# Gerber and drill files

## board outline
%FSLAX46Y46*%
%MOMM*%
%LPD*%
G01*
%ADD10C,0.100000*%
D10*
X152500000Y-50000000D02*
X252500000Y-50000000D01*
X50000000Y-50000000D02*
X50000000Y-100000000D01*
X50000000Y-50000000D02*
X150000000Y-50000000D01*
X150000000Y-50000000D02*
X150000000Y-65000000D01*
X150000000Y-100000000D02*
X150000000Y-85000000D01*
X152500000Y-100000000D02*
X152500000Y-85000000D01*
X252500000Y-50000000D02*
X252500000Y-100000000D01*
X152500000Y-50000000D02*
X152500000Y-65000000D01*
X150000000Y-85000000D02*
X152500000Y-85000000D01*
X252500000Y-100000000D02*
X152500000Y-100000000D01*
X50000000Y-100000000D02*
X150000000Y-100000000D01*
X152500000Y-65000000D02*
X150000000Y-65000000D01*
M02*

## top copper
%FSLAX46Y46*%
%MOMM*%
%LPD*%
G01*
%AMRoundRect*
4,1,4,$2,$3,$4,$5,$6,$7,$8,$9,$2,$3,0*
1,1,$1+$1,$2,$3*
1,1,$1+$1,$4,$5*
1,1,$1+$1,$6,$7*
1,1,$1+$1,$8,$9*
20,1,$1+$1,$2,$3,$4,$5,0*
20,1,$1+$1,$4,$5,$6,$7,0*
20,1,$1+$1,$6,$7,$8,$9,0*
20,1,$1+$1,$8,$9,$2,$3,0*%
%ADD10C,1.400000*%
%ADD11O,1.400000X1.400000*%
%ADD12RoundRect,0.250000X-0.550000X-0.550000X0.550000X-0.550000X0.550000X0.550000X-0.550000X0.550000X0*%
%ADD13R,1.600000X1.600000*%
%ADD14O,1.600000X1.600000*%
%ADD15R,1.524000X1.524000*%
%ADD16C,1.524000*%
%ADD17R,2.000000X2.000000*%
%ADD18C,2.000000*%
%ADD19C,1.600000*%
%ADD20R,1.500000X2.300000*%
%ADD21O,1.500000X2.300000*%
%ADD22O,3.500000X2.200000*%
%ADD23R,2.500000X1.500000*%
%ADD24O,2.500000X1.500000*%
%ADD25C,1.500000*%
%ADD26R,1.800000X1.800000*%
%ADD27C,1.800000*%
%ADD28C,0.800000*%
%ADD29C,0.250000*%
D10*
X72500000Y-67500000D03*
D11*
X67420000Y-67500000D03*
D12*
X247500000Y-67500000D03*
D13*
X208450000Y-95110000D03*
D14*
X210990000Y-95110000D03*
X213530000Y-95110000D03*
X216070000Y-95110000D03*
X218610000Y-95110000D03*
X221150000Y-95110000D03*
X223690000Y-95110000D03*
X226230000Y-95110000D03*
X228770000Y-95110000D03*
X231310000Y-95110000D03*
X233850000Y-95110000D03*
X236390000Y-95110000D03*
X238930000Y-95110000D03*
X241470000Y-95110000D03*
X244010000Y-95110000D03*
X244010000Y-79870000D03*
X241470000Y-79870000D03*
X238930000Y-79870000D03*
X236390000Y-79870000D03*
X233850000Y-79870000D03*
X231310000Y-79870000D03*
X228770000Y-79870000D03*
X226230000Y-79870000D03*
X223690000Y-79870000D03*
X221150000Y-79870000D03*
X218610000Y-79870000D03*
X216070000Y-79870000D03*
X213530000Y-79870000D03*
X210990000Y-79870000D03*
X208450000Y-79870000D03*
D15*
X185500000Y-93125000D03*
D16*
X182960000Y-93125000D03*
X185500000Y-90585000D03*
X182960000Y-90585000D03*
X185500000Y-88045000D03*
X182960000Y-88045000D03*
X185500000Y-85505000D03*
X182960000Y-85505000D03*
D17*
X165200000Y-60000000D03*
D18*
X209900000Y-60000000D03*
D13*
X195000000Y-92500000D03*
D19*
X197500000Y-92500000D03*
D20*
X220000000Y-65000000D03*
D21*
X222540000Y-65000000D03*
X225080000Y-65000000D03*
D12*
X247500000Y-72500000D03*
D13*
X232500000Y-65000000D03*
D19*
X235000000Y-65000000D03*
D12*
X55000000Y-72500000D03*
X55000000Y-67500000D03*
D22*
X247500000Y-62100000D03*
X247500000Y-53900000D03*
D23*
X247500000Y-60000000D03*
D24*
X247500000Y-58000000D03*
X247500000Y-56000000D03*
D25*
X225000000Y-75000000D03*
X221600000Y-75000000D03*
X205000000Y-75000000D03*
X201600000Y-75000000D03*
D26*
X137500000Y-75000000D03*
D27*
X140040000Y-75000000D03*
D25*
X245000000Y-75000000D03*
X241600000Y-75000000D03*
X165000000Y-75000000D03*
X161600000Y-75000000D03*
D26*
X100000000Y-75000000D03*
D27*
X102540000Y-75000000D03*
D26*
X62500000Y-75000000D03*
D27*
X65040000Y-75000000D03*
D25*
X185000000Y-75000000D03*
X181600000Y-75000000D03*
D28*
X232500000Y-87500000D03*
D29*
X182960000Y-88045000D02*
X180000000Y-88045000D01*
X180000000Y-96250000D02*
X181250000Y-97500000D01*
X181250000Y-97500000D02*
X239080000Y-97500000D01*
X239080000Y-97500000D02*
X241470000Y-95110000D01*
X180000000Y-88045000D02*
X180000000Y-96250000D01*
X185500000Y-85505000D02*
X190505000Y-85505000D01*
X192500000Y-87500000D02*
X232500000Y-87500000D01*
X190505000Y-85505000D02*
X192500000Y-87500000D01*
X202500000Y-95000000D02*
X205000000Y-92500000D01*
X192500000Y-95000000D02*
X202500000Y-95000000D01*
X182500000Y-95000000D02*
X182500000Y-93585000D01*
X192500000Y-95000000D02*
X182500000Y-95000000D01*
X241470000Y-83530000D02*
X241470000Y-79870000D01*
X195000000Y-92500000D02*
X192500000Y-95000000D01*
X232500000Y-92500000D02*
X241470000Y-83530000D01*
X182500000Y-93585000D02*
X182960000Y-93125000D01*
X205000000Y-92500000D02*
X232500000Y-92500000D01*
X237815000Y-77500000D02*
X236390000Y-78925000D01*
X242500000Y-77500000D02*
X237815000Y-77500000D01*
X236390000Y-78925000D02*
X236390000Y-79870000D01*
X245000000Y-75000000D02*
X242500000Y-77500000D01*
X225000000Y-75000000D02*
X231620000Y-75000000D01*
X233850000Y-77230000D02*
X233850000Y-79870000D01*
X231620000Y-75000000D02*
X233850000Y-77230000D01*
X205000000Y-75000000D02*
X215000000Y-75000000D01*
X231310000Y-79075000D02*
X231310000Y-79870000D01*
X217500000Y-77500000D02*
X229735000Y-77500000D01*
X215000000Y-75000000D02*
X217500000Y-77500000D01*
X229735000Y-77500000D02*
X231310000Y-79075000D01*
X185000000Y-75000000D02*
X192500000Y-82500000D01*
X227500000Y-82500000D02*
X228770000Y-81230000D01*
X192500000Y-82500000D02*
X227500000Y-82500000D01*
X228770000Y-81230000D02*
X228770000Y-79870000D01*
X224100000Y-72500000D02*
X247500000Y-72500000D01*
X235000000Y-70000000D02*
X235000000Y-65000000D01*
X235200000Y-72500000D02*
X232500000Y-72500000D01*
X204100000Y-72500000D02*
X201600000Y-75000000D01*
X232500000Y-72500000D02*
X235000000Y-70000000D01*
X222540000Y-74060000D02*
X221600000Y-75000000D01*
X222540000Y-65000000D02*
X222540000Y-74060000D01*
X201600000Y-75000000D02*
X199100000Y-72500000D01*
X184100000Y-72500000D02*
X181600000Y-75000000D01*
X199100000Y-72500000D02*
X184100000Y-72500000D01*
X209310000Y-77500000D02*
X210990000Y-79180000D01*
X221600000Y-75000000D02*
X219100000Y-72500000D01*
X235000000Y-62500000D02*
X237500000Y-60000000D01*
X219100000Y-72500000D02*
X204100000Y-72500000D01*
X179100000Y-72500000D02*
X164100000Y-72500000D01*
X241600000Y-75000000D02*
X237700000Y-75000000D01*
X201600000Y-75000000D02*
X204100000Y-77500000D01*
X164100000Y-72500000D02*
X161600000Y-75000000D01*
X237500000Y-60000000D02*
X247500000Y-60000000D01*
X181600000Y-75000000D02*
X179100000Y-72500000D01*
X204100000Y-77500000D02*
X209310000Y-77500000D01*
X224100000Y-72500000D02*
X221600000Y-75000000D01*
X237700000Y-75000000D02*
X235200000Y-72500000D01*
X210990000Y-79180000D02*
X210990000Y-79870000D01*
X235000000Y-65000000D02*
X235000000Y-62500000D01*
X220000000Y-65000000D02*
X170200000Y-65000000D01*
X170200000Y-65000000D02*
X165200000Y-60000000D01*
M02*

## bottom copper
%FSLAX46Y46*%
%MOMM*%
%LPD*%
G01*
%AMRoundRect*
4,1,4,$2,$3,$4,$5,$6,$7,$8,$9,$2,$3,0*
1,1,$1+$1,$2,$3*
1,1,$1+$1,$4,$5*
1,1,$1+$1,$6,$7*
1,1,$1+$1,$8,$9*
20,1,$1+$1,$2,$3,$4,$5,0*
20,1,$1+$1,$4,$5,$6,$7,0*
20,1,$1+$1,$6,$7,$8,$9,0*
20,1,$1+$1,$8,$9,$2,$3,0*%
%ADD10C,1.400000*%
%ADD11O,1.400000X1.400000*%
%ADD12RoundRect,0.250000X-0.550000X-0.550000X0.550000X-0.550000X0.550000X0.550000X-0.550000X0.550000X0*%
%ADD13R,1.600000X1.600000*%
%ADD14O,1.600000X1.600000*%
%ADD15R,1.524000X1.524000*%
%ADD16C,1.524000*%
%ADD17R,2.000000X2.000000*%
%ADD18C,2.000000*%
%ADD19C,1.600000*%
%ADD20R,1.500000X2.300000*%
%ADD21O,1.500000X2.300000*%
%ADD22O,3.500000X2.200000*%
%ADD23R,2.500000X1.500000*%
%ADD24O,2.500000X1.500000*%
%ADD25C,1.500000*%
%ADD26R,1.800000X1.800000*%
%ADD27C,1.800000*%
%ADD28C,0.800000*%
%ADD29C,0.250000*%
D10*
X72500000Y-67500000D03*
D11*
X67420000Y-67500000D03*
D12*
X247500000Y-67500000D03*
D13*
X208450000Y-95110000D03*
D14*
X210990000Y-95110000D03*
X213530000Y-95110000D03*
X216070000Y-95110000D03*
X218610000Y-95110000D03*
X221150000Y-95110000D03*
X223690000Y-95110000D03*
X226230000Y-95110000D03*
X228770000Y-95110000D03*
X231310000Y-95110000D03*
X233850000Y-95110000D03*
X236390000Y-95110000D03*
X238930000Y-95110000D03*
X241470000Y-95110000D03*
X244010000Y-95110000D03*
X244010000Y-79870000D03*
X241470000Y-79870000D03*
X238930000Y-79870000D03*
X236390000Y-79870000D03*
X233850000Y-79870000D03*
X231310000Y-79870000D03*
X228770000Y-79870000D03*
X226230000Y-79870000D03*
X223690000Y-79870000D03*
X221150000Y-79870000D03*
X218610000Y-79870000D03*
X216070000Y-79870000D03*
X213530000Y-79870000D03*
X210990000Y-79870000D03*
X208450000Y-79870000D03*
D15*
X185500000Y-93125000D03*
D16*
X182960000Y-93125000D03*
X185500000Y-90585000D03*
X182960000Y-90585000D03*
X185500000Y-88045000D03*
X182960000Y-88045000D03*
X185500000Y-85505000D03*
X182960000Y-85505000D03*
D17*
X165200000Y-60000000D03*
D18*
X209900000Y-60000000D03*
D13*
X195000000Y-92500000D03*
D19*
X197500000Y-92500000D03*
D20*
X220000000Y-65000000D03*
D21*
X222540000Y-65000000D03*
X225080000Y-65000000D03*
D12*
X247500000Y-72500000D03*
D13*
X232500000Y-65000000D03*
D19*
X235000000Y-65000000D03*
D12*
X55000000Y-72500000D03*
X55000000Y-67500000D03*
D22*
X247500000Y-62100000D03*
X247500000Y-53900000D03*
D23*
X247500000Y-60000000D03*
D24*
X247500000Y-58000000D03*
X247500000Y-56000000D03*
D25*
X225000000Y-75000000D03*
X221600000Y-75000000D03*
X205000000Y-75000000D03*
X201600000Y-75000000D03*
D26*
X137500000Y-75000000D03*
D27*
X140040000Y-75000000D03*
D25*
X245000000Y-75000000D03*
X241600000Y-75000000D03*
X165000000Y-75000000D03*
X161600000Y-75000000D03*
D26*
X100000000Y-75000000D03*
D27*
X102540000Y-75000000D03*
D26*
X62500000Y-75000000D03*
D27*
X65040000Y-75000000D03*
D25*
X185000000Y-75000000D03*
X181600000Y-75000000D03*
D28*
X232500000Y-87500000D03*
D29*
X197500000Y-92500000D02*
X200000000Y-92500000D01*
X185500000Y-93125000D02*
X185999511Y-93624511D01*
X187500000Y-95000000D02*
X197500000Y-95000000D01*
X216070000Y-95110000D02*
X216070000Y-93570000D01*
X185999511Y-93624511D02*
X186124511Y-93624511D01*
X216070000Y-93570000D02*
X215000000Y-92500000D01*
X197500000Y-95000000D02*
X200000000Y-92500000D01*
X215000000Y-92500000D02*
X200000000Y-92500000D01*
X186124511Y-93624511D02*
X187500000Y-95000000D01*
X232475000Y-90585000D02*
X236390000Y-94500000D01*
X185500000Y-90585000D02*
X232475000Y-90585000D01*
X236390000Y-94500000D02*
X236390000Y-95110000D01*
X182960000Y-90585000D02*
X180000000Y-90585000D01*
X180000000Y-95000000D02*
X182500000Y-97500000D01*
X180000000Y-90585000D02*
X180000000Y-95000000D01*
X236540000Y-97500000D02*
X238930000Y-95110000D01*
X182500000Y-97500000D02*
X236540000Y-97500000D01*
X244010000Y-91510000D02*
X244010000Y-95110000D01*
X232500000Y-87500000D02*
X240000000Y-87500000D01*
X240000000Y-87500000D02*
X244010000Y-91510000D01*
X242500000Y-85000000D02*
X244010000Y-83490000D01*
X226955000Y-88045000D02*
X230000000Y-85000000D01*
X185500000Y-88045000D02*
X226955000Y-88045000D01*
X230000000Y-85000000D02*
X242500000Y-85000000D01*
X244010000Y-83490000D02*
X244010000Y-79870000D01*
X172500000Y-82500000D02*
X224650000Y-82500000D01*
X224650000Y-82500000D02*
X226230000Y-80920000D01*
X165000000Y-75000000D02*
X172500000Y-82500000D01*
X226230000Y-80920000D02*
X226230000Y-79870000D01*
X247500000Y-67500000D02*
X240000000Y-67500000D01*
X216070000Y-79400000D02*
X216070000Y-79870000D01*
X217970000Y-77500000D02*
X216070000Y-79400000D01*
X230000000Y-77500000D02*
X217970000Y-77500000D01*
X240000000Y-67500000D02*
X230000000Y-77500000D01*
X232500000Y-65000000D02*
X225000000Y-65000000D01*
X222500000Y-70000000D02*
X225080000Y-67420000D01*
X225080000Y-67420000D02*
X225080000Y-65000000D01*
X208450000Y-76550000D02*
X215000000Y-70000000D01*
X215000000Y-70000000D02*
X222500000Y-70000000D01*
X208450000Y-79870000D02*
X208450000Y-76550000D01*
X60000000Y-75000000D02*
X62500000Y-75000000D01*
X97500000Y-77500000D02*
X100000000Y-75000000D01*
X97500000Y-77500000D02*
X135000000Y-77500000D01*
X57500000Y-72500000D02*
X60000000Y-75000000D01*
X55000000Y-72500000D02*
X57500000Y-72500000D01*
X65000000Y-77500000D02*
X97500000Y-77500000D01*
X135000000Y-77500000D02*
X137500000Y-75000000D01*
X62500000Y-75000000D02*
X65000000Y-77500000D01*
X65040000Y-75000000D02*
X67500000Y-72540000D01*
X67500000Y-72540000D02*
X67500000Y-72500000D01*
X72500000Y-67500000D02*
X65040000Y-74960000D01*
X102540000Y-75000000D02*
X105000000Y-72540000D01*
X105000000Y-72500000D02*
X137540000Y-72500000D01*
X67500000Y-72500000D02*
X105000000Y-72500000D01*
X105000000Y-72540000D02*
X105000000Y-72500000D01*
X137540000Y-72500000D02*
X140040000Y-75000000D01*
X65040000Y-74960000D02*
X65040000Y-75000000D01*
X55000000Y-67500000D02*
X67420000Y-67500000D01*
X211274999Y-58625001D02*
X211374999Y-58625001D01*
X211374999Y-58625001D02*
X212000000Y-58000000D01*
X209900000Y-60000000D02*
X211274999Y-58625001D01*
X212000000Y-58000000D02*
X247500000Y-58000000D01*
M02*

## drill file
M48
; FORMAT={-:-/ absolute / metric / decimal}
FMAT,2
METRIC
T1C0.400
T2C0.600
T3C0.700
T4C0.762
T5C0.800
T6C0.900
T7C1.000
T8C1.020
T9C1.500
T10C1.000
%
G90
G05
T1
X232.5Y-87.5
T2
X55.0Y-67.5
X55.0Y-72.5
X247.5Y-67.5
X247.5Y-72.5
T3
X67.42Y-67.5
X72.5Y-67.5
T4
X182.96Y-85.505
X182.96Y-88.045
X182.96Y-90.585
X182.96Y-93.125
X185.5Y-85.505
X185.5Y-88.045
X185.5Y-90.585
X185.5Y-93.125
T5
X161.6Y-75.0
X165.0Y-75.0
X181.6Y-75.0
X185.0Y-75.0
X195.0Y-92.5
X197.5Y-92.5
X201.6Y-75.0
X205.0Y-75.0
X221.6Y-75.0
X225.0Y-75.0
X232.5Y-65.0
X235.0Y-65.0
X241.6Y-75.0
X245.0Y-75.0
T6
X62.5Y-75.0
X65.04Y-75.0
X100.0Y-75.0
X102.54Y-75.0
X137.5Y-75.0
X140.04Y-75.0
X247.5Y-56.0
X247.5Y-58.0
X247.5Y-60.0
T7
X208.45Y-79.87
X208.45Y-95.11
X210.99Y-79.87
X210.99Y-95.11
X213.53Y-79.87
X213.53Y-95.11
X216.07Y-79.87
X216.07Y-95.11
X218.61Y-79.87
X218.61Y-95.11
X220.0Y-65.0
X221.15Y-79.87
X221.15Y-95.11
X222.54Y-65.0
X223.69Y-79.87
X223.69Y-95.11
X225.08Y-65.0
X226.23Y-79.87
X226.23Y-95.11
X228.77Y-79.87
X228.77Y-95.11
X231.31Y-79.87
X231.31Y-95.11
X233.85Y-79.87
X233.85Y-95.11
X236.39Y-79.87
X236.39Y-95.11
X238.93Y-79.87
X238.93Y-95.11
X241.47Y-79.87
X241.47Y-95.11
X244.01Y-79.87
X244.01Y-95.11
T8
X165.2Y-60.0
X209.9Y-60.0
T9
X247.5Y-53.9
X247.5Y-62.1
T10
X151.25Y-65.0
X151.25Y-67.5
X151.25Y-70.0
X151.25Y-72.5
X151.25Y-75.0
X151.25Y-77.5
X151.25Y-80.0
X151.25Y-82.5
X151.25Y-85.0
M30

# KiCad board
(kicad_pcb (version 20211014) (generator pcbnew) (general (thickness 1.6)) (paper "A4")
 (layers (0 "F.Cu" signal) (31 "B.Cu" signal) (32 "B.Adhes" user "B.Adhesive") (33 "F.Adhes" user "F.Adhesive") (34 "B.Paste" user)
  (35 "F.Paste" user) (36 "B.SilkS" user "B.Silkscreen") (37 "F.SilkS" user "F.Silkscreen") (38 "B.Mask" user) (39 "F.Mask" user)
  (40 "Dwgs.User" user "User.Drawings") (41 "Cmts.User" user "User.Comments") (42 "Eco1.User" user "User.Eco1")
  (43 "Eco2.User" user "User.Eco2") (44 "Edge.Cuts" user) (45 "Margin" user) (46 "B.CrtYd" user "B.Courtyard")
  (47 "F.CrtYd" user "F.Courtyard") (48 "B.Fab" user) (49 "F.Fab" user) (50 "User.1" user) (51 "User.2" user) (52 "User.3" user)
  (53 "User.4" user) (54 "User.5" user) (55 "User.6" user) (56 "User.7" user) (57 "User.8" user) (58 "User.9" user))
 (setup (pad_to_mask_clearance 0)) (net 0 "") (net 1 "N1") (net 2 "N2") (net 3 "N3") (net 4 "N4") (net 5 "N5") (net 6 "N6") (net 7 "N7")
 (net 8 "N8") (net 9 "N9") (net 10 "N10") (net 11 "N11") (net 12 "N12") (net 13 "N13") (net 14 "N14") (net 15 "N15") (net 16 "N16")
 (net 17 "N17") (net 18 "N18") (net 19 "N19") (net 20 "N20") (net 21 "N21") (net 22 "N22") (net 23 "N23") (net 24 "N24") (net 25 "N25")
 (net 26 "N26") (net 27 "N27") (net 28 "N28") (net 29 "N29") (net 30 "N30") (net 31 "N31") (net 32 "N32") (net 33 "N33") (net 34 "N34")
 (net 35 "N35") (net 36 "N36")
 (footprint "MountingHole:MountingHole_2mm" (layer "F.Cu") (at 151.25 72.5)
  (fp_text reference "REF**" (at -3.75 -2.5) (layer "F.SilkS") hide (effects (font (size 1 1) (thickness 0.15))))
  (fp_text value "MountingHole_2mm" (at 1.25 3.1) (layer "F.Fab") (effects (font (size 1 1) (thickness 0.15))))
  (pad "" np_thru_hole circle (at 0 0) (size 1 1) (drill 1) (layers F&B.Cu *.Mask)))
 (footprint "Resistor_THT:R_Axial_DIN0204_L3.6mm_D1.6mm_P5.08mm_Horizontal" (layer "F.Cu") (at 72.5 67.5 180)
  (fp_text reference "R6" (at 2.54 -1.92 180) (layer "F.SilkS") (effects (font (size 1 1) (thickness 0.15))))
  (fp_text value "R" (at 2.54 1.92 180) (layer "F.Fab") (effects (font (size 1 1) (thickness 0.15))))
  (pad "1" thru_hole circle (at 0 0 180) (size 1.4 1.4) (drill 0.7) (layers *.Cu *.Mask) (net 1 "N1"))
  (pad "2" thru_hole oval (at 5.08 0 180) (size 1.4 1.4) (drill 0.7) (layers *.Cu *.Mask) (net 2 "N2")))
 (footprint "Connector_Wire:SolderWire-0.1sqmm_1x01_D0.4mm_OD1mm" (layer "F.Cu") (at 247.5 67.5)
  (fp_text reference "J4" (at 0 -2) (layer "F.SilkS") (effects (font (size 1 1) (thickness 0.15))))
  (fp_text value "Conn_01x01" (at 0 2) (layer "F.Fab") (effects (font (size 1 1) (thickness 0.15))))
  (pad "1" thru_hole roundrect (at 0 0) (size 1.6 1.6) (drill 0.6) (layers *.Cu *.Mask) (roundrect_rratio 0.15625) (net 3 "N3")))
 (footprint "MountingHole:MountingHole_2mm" (layer "F.Cu") (at 151.25 77.5)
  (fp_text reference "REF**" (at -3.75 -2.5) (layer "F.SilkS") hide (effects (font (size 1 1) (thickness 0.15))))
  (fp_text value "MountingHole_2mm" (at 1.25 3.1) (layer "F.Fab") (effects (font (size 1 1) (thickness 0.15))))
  (pad "" np_thru_hole circle (at 0 0) (size 1 1) (drill 1) (layers F&B.Cu *.Mask)))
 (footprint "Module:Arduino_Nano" (layer "F.Cu") (at 208.45 95.11 90)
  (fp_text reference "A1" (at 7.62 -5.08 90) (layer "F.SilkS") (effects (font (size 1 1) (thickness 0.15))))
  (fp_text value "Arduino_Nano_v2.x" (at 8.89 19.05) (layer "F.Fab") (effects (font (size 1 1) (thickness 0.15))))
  (pad "1" thru_hole rect (at 0 0 90) (size 1.6 1.6) (drill 1) (layers *.Cu *.Mask) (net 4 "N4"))
  (pad "2" thru_hole oval (at 0 2.54 90) (size 1.6 1.6) (drill 1) (layers *.Cu *.Mask) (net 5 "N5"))
  (pad "3" thru_hole oval (at 0 5.08 90) (size 1.6 1.6) (drill 1) (layers *.Cu *.Mask) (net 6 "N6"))
  (pad "4" thru_hole oval (at 0 7.62 90) (size 1.6 1.6) (drill 1) (layers *.Cu *.Mask) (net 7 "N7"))
  (pad "5" thru_hole oval (at 0 10.16 90) (size 1.6 1.6) (drill 1) (layers *.Cu *.Mask) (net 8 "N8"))
  (pad "6" thru_hole oval (at 0 12.7 90) (size 1.6 1.6) (drill 1) (layers *.Cu *.Mask) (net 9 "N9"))
  (pad "7" thru_hole oval (at 0 15.24 90) (size 1.6 1.6) (drill 1) (layers *.Cu *.Mask) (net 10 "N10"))
  (pad "8" thru_hole oval (at 0 17.78 90) (size 1.6 1.6) (drill 1) (layers *.Cu *.Mask) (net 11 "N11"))
  (pad "9" thru_hole oval (at 0 20.32 90) (size 1.6 1.6) (drill 1) (layers *.Cu *.Mask) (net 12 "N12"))
  (pad "10" thru_hole oval (at 0 22.86 90) (size 1.6 1.6) (drill 1) (layers *.Cu *.Mask) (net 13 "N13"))
  (pad "11" thru_hole oval (at 0 25.4 90) (size 1.6 1.6) (drill 1) (layers *.Cu *.Mask) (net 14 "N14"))
  (pad "12" thru_hole oval (at 0 27.94 90) (size 1.6 1.6) (drill 1) (layers *.Cu *.Mask) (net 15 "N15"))
  (pad "13" thru_hole oval (at 0 30.48 90) (size 1.6 1.6) (drill 1) (layers *.Cu *.Mask) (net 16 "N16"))
  (pad "14" thru_hole oval (at 0 33.02 90) (size 1.6 1.6) (drill 1) (layers *.Cu *.Mask) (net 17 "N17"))
  (pad "15" thru_hole oval (at 0 35.56 90) (size 1.6 1.6) (drill 1) (layers *.Cu *.Mask) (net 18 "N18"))
  (pad "16" thru_hole oval (at 15.24 35.56 90) (size 1.6 1.6) (drill 1) (layers *.Cu *.Mask) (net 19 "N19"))
  (pad "17" thru_hole oval (at 15.24 33.02 90) (size 1.6 1.6) (drill 1) (layers *.Cu *.Mask) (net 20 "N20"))
  (pad "18" thru_hole oval (at 15.24 30.48 90) (size 1.6 1.6) (drill 1) (layers *.Cu *.Mask) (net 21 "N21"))
  (pad "19" thru_hole oval (at 15.24 27.94 90) (size 1.6 1.6) (drill 1) (layers *.Cu *.Mask) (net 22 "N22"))
  (pad "20" thru_hole oval (at 15.24 25.4 90) (size 1.6 1.6) (drill 1) (layers *.Cu *.Mask) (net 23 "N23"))
  (pad "21" thru_hole oval (at 15.24 22.86 90) (size 1.6 1.6) (drill 1) (layers *.Cu *.Mask) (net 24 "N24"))
  (pad "22" thru_hole oval (at 15.24 20.32 90) (size 1.6 1.6) (drill 1) (layers *.Cu *.Mask) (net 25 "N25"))
  (pad "23" thru_hole oval (at 15.24 17.78 90) (size 1.6 1.6) (drill 1) (layers *.Cu *.Mask) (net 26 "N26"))
  (pad "24" thru_hole oval (at 15.24 15.24 90) (size 1.6 1.6) (drill 1) (layers *.Cu *.Mask) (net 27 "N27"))
  (pad "25" thru_hole oval (at 15.24 12.7 90) (size 1.6 1.6) (drill 1) (layers *.Cu *.Mask) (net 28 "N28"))
  (pad "26" thru_hole oval (at 15.24 10.16 90) (size 1.6 1.6) (drill 1) (layers *.Cu *.Mask) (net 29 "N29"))
  (pad "27" thru_hole oval (at 15.24 7.62 90) (size 1.6 1.6) (drill 1) (layers *.Cu *.Mask) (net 3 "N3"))
  (pad "28" thru_hole oval (at 15.24 5.08 90) (size 1.6 1.6) (drill 1) (layers *.Cu *.Mask) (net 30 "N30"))
  (pad "29" thru_hole oval (at 15.24 2.54 90) (size 1.6 1.6) (drill 1) (layers *.Cu *.Mask) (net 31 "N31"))
  (pad "30" thru_hole oval (at 15.24 0 90) (size 1.6 1.6) (drill 1) (layers *.Cu *.Mask) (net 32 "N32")))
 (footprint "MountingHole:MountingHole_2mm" (layer "F.Cu") (at 151.25 65)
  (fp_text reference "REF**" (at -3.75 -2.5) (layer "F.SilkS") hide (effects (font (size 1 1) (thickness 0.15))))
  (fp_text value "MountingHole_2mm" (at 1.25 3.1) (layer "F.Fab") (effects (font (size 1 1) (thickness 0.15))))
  (pad "" np_thru_hole circle (at 0 0) (size 1 1) (drill 1) (layers F&B.Cu *.Mask)))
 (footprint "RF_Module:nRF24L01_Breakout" (layer "F.Cu") (at 185.5 93.125 180)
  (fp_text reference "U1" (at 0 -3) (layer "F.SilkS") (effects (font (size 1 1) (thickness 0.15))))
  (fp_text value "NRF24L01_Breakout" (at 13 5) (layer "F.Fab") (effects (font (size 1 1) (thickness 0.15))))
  (pad "1" thru_hole rect (at 0 0 180) (size 1.524 1.524) (drill 0.762) (layers *.Cu *.Mask) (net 7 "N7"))
  (pad "2" thru_hole circle (at 2.54 0 180) (size 1.524 1.524) (drill 0.762) (layers *.Cu *.Mask) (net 20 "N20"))
  (pad "3" thru_hole circle (at 0 2.54 180) (size 1.524 1.524) (drill 0.762) (layers *.Cu *.Mask) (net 15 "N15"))
  (pad "4" thru_hole circle (at 2.54 2.54 180) (size 1.524 1.524) (drill 0.762) (layers *.Cu *.Mask) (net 16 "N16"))
  (pad "5" thru_hole circle (at 0 5.08 180) (size 1.524 1.524) (drill 0.762) (layers *.Cu *.Mask) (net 19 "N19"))
  (pad "6" thru_hole circle (at 2.54 5.08 180) (size 1.524 1.524) (drill 0.762) (layers *.Cu *.Mask) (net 17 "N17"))
  (pad "7" thru_hole circle (at 0 7.62 180) (size 1.524 1.524) (drill 0.762) (layers *.Cu *.Mask) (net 18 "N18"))
  (pad "8" thru_hole circle (at 2.54 7.62 180) (size 1.524 1.524) (drill 0.762) (layers *.Cu *.Mask) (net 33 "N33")))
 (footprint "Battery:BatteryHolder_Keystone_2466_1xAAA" (layer "F.Cu") (at 165.2 60)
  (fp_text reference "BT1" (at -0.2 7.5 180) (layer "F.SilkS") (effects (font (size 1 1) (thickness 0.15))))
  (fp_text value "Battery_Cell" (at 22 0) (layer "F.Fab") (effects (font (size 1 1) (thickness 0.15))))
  (pad "1" thru_hole rect (at 0 0) (size 2 2) (drill 1.02) (layers *.Cu *.Mask) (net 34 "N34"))
  (pad "2" thru_hole circle (at 44.7 0) (size 2 2) (drill 1.02) (layers *.Cu *.Mask) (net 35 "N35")))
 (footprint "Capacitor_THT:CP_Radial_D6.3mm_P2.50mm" (layer "F.Cu") (at 195 92.5)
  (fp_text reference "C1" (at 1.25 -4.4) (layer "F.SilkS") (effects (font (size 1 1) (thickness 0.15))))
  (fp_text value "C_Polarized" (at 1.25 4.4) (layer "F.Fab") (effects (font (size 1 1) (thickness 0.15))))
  (pad "1" thru_hole rect (at 0 0) (size 1.6 1.6) (drill 0.8) (layers *.Cu *.Mask) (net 20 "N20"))
  (pad "2" thru_hole circle (at 2.5 0) (size 1.6 1.6) (drill 0.8) (layers *.Cu *.Mask) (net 7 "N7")))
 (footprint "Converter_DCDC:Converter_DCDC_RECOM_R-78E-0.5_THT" (layer "F.Cu") (at 220 65)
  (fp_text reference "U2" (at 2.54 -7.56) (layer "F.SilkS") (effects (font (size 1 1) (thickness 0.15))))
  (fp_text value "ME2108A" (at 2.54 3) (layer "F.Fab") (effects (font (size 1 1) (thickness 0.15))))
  (pad "1" thru_hole rect (at 0 0) (size 1.5 2.3) (drill 1) (layers *.Cu *.Mask) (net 34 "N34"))
  (pad "2" thru_hole oval (at 2.54 0) (size 1.5 2.3) (drill 1) (layers *.Cu *.Mask) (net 31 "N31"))
  (pad "3" thru_hole oval (at 5.08 0) (size 1.5 2.3) (drill 1) (layers *.Cu *.Mask) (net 32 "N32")))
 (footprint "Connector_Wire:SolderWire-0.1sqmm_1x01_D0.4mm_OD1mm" (layer "F.Cu") (at 247.5 72.5)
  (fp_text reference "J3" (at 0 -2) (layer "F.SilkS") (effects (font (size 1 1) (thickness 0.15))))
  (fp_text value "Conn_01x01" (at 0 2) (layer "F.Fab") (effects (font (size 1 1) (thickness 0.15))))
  (pad "1" thru_hole roundrect (at 0 0) (size 1.6 1.6) (drill 0.6) (layers *.Cu *.Mask) (roundrect_rratio 0.15625) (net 31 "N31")))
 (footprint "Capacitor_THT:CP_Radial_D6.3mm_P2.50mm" (layer "F.Cu") (at 232.5 65)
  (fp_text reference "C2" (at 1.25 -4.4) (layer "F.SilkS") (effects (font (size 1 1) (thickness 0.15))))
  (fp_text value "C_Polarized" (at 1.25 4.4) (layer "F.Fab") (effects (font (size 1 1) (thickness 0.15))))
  (pad "1" thru_hole rect (at 0 0) (size 1.6 1.6) (drill 0.8) (layers *.Cu *.Mask) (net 32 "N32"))
  (pad "2" thru_hole circle (at 2.5 0) (size 1.6 1.6) (drill 0.8) (layers *.Cu *.Mask) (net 31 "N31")))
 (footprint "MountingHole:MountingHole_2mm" (layer "F.Cu") (at 151.25 80)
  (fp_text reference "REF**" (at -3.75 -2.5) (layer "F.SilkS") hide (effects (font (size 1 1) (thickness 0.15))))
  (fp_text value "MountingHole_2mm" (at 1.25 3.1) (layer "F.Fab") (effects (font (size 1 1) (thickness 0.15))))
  (pad "" np_thru_hole circle (at 0 0) (size 1 1) (drill 1) (layers F&B.Cu *.Mask)))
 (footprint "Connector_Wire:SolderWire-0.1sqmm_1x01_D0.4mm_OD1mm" (layer "F.Cu") (at 55 72.5)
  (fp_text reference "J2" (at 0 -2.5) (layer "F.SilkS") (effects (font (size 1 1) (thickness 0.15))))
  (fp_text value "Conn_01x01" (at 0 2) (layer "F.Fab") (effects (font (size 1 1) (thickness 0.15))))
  (pad "1" thru_hole roundrect (at 0 0) (size 1.6 1.6) (drill 0.6) (layers *.Cu *.Mask) (roundrect_rratio 0.15625) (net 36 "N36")))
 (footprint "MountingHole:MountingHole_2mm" (layer "F.Cu") (at 151.25 85)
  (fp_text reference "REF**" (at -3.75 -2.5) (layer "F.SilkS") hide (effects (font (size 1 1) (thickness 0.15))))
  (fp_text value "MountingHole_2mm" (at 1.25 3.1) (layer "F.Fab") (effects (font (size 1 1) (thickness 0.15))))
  (pad "" np_thru_hole circle (at 0 0) (size 1 1) (drill 1) (layers F&B.Cu *.Mask)))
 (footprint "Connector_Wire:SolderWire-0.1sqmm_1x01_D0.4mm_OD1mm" (layer "F.Cu") (at 55 67.5)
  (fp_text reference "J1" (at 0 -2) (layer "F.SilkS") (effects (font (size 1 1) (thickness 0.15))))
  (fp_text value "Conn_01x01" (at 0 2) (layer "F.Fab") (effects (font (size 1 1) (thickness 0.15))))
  (pad "1" thru_hole roundrect (at 0 0) (size 1.6 1.6) (drill 0.6) (layers *.Cu *.Mask) (roundrect_rratio 0.15625) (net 2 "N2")))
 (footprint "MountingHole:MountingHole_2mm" (layer "F.Cu") (at 151.25 67.5)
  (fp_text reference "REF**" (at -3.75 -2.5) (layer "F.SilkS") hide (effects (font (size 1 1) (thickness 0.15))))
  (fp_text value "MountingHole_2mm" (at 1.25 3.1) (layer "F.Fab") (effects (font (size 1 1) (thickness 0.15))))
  (pad "" np_thru_hole circle (at 0 0) (size 1 1) (drill 1) (layers F&B.Cu *.Mask)))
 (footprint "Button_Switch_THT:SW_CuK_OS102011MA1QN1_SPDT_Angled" (layer "F.Cu") (at 247.5 60 90)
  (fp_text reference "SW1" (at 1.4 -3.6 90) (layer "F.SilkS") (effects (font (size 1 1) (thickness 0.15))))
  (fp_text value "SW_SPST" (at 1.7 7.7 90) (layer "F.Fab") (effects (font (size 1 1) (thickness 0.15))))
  (pad "" thru_hole oval (at -2.1 0 90) (size 2.2 3.5) (drill 1.5) (layers *.Cu *.Mask))
  (pad "" thru_hole oval (at 6.1 0 90) (size 2.2 3.5) (drill 1.5) (layers *.Cu *.Mask))
  (pad "1" thru_hole rect (at 0 0 90) (size 1.5 2.5) (drill 0.9) (layers *.Cu *.Mask) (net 31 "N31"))
  (pad "2" thru_hole oval (at 2 0 90) (size 1.5 2.5) (drill 0.9) (layers *.Cu *.Mask) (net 35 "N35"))
  (pad "3" thru_hole oval (at 4 0 90) (size 1.5 2.5) (drill 0.9) (layers *.Cu *.Mask)))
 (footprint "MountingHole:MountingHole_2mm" (layer "F.Cu") (at 151.25 75)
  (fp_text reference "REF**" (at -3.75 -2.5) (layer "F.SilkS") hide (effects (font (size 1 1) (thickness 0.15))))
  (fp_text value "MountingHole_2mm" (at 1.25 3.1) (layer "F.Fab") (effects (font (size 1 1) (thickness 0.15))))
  (pad "" np_thru_hole circle (at 0 0) (size 1 1) (drill 1) (layers F&B.Cu *.Mask)))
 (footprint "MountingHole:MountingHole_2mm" (layer "F.Cu") (at 151.25 70)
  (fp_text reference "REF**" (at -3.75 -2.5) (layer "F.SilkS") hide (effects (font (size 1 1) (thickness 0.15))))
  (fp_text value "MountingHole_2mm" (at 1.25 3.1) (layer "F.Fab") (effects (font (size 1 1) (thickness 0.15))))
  (pad "" np_thru_hole circle (at 0 0) (size 1 1) (drill 1) (layers F&B.Cu *.Mask)))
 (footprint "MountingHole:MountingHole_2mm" (layer "F.Cu") (at 151.25 82.5)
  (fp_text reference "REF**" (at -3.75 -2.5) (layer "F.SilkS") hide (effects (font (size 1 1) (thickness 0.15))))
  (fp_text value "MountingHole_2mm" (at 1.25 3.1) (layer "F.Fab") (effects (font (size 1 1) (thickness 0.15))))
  (pad "" np_thru_hole circle (at 0 0) (size 1 1) (drill 1) (layers F&B.Cu *.Mask)))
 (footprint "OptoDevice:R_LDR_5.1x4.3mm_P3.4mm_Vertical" (layer "B.Cu") (at 225 75 180)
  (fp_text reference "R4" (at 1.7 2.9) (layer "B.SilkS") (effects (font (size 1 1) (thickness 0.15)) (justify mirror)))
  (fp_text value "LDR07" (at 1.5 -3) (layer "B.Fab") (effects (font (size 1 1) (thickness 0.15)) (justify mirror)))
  (pad "1" thru_hole circle (at 0 0 180) (size 1.5 1.5) (drill 0.8) (layers *.Cu *.Mask) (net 23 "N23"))
  (pad "2" thru_hole circle (at 3.4 0 180) (size 1.5 1.5) (drill 0.8) (layers *.Cu *.Mask) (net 31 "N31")))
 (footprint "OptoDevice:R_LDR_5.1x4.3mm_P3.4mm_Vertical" (layer "B.Cu") (at 205 75 180)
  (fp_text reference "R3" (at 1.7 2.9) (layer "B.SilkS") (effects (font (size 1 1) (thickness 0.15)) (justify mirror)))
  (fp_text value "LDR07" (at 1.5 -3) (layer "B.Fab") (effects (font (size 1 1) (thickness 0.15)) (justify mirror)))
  (pad "1" thru_hole circle (at 0 0 180) (size 1.5 1.5) (drill 0.8) (layers *.Cu *.Mask) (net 24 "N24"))
  (pad "2" thru_hole circle (at 3.4 0 180) (size 1.5 1.5) (drill 0.8) (layers *.Cu *.Mask) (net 31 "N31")))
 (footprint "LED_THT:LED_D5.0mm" (layer "B.Cu") (at 137.5 75)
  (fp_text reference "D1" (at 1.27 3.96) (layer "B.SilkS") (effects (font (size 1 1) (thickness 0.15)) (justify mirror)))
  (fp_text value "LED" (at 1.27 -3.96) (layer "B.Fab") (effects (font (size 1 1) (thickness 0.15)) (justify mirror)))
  (pad "1" thru_hole rect (at 0 0) (size 1.8 1.8) (drill 0.9) (layers *.Cu *.Mask) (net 36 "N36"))
  (pad "2" thru_hole circle (at 2.54 0) (size 1.8 1.8) (drill 0.9) (layers *.Cu *.Mask) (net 1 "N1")))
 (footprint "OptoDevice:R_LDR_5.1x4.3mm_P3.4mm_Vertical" (layer "B.Cu") (at 245 75 180)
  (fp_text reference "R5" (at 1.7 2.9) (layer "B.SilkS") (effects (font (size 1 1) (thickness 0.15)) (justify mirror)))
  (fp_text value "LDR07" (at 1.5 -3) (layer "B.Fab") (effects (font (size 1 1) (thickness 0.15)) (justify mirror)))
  (pad "1" thru_hole circle (at 0 0 180) (size 1.5 1.5) (drill 0.8) (layers *.Cu *.Mask) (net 22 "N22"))
  (pad "2" thru_hole circle (at 3.4 0 180) (size 1.5 1.5) (drill 0.8) (layers *.Cu *.Mask) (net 31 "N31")))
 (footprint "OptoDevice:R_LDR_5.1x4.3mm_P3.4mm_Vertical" (layer "B.Cu") (at 165 75 180)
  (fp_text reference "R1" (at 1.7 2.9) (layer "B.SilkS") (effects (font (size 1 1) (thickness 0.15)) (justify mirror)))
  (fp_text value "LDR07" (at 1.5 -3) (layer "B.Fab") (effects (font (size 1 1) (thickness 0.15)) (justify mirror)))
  (pad "1" thru_hole circle (at 0 0 180) (size 1.5 1.5) (drill 0.8) (layers *.Cu *.Mask) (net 26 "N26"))
  (pad "2" thru_hole circle (at 3.4 0 180) (size 1.5 1.5) (drill 0.8) (layers *.Cu *.Mask) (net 31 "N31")))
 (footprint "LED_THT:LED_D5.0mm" (layer "B.Cu") (at 100 75)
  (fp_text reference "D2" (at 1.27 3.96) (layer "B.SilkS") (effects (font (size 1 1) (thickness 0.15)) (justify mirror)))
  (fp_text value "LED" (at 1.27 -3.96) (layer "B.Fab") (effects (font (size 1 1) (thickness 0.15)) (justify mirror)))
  (pad "1" thru_hole rect (at 0 0) (size 1.8 1.8) (drill 0.9) (layers *.Cu *.Mask) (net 36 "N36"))
  (pad "2" thru_hole circle (at 2.54 0) (size 1.8 1.8) (drill 0.9) (layers *.Cu *.Mask) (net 1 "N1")))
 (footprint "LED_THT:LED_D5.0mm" (layer "B.Cu") (at 62.5 75)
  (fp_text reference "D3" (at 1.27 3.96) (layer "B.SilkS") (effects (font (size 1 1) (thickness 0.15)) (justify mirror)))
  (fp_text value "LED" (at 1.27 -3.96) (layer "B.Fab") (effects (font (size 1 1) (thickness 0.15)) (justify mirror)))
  (pad "1" thru_hole rect (at 0 0) (size 1.8 1.8) (drill 0.9) (layers *.Cu *.Mask) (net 36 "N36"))
  (pad "2" thru_hole circle (at 2.54 0) (size 1.8 1.8) (drill 0.9) (layers *.Cu *.Mask) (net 1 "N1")))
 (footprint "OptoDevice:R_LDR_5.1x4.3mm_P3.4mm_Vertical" (layer "B.Cu") (at 185 75 180)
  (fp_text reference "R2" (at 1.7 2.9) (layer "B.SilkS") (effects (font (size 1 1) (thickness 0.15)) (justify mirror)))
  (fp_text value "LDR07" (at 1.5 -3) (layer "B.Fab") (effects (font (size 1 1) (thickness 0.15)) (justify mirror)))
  (pad "1" thru_hole circle (at 0 0 180) (size 1.5 1.5) (drill 0.8) (layers *.Cu *.Mask) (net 25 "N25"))
  (pad "2" thru_hole circle (at 3.4 0 180) (size 1.5 1.5) (drill 0.8) (layers *.Cu *.Mask) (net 31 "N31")))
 (gr_line (start 152.5 50) (end 252.5 50) (layer "Edge.Cuts") (width 0.1))
 (gr_line (start 50 50) (end 50 100) (layer "Edge.Cuts") (width 0.1))
 (gr_line (start 50 50) (end 150 50) (layer "Edge.Cuts") (width 0.1))
 (gr_line (start 150 50) (end 150 65) (layer "Edge.Cuts") (width 0.1))
 (gr_line (start 150 100) (end 150 85) (layer "Edge.Cuts") (width 0.1))
 (gr_line (start 152.5 100) (end 152.5 85) (layer "Edge.Cuts") (width 0.1))
 (gr_line (start 252.5 50) (end 252.5 100) (layer "Edge.Cuts") (width 0.1))
 (gr_line (start 152.5 50) (end 152.5 65) (layer "Edge.Cuts") (width 0.1))
 (gr_line (start 150 85) (end 152.5 85) (layer "Edge.Cuts") (width 0.1))
 (gr_line (start 252.5 100) (end 152.5 100) (layer "Edge.Cuts") (width 0.1))
 (gr_line (start 50 100) (end 150 100) (layer "Edge.Cuts") (width 0.1))
 (gr_line (start 152.5 65) (end 150 65) (layer "Edge.Cuts") (width 0.1))
 (segment (start 197.5 92.5) (end 200 92.5) (width 0.25) (layer "B.Cu") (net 7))
 (segment (start 185.5 93.125) (end 185.999511 93.624511) (width 0.25) (layer "B.Cu") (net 7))
 (segment (start 187.5 95) (end 197.5 95) (width 0.25) (layer "B.Cu") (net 7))
 (segment (start 216.07 95.11) (end 216.07 93.57) (width 0.25) (layer "B.Cu") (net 7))
 (segment (start 185.999511 93.624511) (end 186.124511 93.624511) (width 0.25) (layer "B.Cu") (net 7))
 (segment (start 216.07 93.57) (end 215 92.5) (width 0.25) (layer "B.Cu") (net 7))
 (segment (start 197.5 95) (end 200 92.5) (width 0.25) (layer "B.Cu") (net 7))
 (segment (start 215 92.5) (end 200 92.5) (width 0.25) (layer "B.Cu") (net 7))
 (segment (start 186.124511 93.624511) (end 187.5 95) (width 0.25) (layer "B.Cu") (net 7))
 (segment (start 232.475 90.585) (end 236.39 94.5) (width 0.25) (layer "B.Cu") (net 15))
 (segment (start 185.5 90.585) (end 232.475 90.585) (width 0.25) (layer "B.Cu") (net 15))
 (segment (start 236.39 94.5) (end 236.39 95.11) (width 0.25) (layer "B.Cu") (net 15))
 (segment (start 182.96 90.585) (end 180 90.585) (width 0.25) (layer "B.Cu") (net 16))
 (segment (start 180 95) (end 182.5 97.5) (width 0.25) (layer "B.Cu") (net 16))
 (segment (start 180 90.585) (end 180 95) (width 0.25) (layer "B.Cu") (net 16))
 (segment (start 236.54 97.5) (end 238.93 95.11) (width 0.25) (layer "B.Cu") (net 16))
 (segment (start 182.5 97.5) (end 236.54 97.5) (width 0.25) (layer "B.Cu") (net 16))
 (segment (start 182.96 88.045) (end 180 88.045) (width 0.25) (layer "F.Cu") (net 17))
 (segment (start 180 96.25) (end 181.25 97.5) (width 0.25) (layer "F.Cu") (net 17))
 (segment (start 181.25 97.5) (end 239.08 97.5) (width 0.25) (layer "F.Cu") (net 17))
 (segment (start 239.08 97.5) (end 241.47 95.11) (width 0.25) (layer "F.Cu") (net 17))
 (segment (start 180 88.045) (end 180 96.25) (width 0.25) (layer "F.Cu") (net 17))
 (segment (start 185.5 85.505) (end 190.505 85.505) (width 0.25) (layer "F.Cu") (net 18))
 (segment (start 192.5 87.5) (end 232.5 87.5) (width 0.25) (layer "F.Cu") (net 18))
 (segment (start 190.505 85.505) (end 192.5 87.5) (width 0.25) (layer "F.Cu") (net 18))
 (via (at 232.5 87.5) (size 0.8) (drill 0.4) (layers "F.Cu" "B.Cu") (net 18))
 (segment (start 244.01 91.51) (end 244.01 95.11) (width 0.25) (layer "B.Cu") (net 18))
 (segment (start 232.5 87.5) (end 240 87.5) (width 0.25) (layer "B.Cu") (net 18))
 (segment (start 240 87.5) (end 244.01 91.51) (width 0.25) (layer "B.Cu") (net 18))
 (segment (start 242.5 85) (end 244.01 83.49) (width 0.25) (layer "B.Cu") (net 19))
 (segment (start 226.955 88.045) (end 230 85) (width 0.25) (layer "B.Cu") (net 19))
 (segment (start 185.5 88.045) (end 226.955 88.045) (width 0.25) (layer "B.Cu") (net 19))
 (segment (start 230 85) (end 242.5 85) (width 0.25) (layer "B.Cu") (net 19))
 (segment (start 244.01 83.49) (end 244.01 79.87) (width 0.25) (layer "B.Cu") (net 19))
 (segment (start 202.5 95) (end 205 92.5) (width 0.25) (layer "F.Cu") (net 20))
 (segment (start 192.5 95) (end 202.5 95) (width 0.25) (layer "F.Cu") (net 20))
 (segment (start 182.5 95) (end 182.5 93.585) (width 0.25) (layer "F.Cu") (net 20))
 (segment (start 192.5 95) (end 182.5 95) (width 0.25) (layer "F.Cu") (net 20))
 (segment (start 241.47 83.53) (end 241.47 79.87) (width 0.25) (layer "F.Cu") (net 20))
 (segment (start 195 92.5) (end 192.5 95) (width 0.25) (layer "F.Cu") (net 20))
 (segment (start 232.5 92.5) (end 241.47 83.53) (width 0.25) (layer "F.Cu") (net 20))
 (segment (start 182.5 93.585) (end 182.96 93.125) (width 0.25) (layer "F.Cu") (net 20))
 (segment (start 205 92.5) (end 232.5 92.5) (width 0.25) (layer "F.Cu") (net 20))
 (segment (start 237.815 77.5) (end 236.39 78.925) (width 0.25) (layer "F.Cu") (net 22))
 (segment (start 242.5 77.5) (end 237.815 77.5) (width 0.25) (layer "F.Cu") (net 22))
 (segment (start 236.39 78.925) (end 236.39 79.87) (width 0.25) (layer "F.Cu") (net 22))
 (segment (start 245 75) (end 242.5 77.5) (width 0.25) (layer "F.Cu") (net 22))
 (segment (start 225 75) (end 231.62 75) (width 0.25) (layer "F.Cu") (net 23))
 (segment (start 233.85 77.23) (end 233.85 79.87) (width 0.25) (layer "F.Cu") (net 23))
 (segment (start 231.62 75) (end 233.85 77.23) (width 0.25) (layer "F.Cu") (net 23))
 (segment (start 205 75) (end 215 75) (width 0.25) (layer "F.Cu") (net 24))
 (segment (start 231.31 79.075) (end 231.31 79.87) (width 0.25) (layer "F.Cu") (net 24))
 (segment (start 217.5 77.5) (end 229.735 77.5) (width 0.25) (layer "F.Cu") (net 24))
 (segment (start 215 75) (end 217.5 77.5) (width 0.25) (layer "F.Cu") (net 24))
 (segment (start 229.735 77.5) (end 231.31 79.075) (width 0.25) (layer "F.Cu") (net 24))
 (segment (start 185 75) (end 192.5 82.5) (width 0.25) (layer "F.Cu") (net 25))
 (segment (start 227.5 82.5) (end 228.77 81.23) (width 0.25) (layer "F.Cu") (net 25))
 (segment (start 192.5 82.5) (end 227.5 82.5) (width 0.25) (layer "F.Cu") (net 25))
 (segment (start 228.77 81.23) (end 228.77 79.87) (width 0.25) (layer "F.Cu") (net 25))
 (segment (start 172.5 82.5) (end 224.65 82.5) (width 0.25) (layer "B.Cu") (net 26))
 (segment (start 224.65 82.5) (end 226.23 80.92) (width 0.25) (layer "B.Cu") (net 26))
 (segment (start 165 75) (end 172.5 82.5) (width 0.25) (layer "B.Cu") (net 26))
 (segment (start 226.23 80.92) (end 226.23 79.87) (width 0.25) (layer "B.Cu") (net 26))
 (segment (start 247.5 67.5) (end 240 67.5) (width 0.25) (layer "B.Cu") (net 3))
 (segment (start 216.07 79.4) (end 216.07 79.87) (width 0.25) (layer "B.Cu") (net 3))
 (segment (start 217.97 77.5) (end 216.07 79.4) (width 0.25) (layer "B.Cu") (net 3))
 (segment (start 230 77.5) (end 217.97 77.5) (width 0.25) (layer "B.Cu") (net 3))
 (segment (start 240 67.5) (end 230 77.5) (width 0.25) (layer "B.Cu") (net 3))
 (segment (start 224.1 72.5) (end 247.5 72.5) (width 0.25) (layer "F.Cu") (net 31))
 (segment (start 235 70) (end 235 65) (width 0.25) (layer "F.Cu") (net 31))
 (segment (start 235.2 72.5) (end 232.5 72.5) (width 0.25) (layer "F.Cu") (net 31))
 (segment (start 204.1 72.5) (end 201.6 75) (width 0.25) (layer "F.Cu") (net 31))
 (segment (start 232.5 72.5) (end 235 70) (width 0.25) (layer "F.Cu") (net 31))
 (segment (start 222.54 74.06) (end 221.6 75) (width 0.25) (layer "F.Cu") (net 31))
 (segment (start 222.54 65) (end 222.54 74.06) (width 0.25) (layer "F.Cu") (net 31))
 (segment (start 201.6 75) (end 199.1 72.5) (width 0.25) (layer "F.Cu") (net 31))
 (segment (start 184.1 72.5) (end 181.6 75) (width 0.25) (layer "F.Cu") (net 31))
 (segment (start 199.1 72.5) (end 184.1 72.5) (width 0.25) (layer "F.Cu") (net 31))
 (segment (start 209.31 77.5) (end 210.99 79.18) (width 0.25) (layer "F.Cu") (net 31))
 (segment (start 221.6 75) (end 219.1 72.5) (width 0.25) (layer "F.Cu") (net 31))
 (segment (start 235 62.5) (end 237.5 60) (width 0.25) (layer "F.Cu") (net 31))
 (segment (start 219.1 72.5) (end 204.1 72.5) (width 0.25) (layer "F.Cu") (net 31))
 (segment (start 179.1 72.5) (end 164.1 72.5) (width 0.25) (layer "F.Cu") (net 31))
 (segment (start 241.6 75) (end 237.7 75) (width 0.25) (layer "F.Cu") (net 31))
 (segment (start 201.6 75) (end 204.1 77.5) (width 0.25) (layer "F.Cu") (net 31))
 (segment (start 164.1 72.5) (end 161.6 75) (width 0.25) (layer "F.Cu") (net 31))
 (segment (start 237.5 60) (end 247.5 60) (width 0.25) (layer "F.Cu") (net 31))
 (segment (start 181.6 75) (end 179.1 72.5) (width 0.25) (layer "F.Cu") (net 31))
 (segment (start 204.1 77.5) (end 209.31 77.5) (width 0.25) (layer "F.Cu") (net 31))
 (segment (start 224.1 72.5) (end 221.6 75) (width 0.25) (layer "F.Cu") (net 31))
 (segment (start 237.7 75) (end 235.2 72.5) (width 0.25) (layer "F.Cu") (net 31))
 (segment (start 210.99 79.18) (end 210.99 79.87) (width 0.25) (layer "F.Cu") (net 31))
 (segment (start 235 65) (end 235 62.5) (width 0.25) (layer "F.Cu") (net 31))
 (segment (start 232.5 65) (end 225 65) (width 0.25) (layer "B.Cu") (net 32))
 (segment (start 222.5 70) (end 225.08 67.42) (width 0.25) (layer "B.Cu") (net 32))
 (segment (start 225.08 67.42) (end 225.08 65) (width 0.25) (layer "B.Cu") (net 32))
 (segment (start 208.45 76.55) (end 215 70) (width 0.25) (layer "B.Cu") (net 32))
 (segment (start 215 70) (end 222.5 70) (width 0.25) (layer "B.Cu") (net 32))
 (segment (start 208.45 79.87) (end 208.45 76.55) (width 0.25) (layer "B.Cu") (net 32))
 (segment (start 60 75) (end 62.5 75) (width 0.25) (layer "B.Cu") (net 36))
 (segment (start 97.5 77.5) (end 100 75) (width 0.25) (layer "B.Cu") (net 36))
 (segment (start 97.5 77.5) (end 135 77.5) (width 0.25) (layer "B.Cu") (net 36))
 (segment (start 57.5 72.5) (end 60 75) (width 0.25) (layer "B.Cu") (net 36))
 (segment (start 55 72.5) (end 57.5 72.5) (width 0.25) (layer "B.Cu") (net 36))
 (segment (start 65 77.5) (end 97.5 77.5) (width 0.25) (layer "B.Cu") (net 36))
 (segment (start 135 77.5) (end 137.5 75) (width 0.25) (layer "B.Cu") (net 36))
 (segment (start 62.5 75) (end 65 77.5) (width 0.25) (layer "B.Cu") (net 36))
 (segment (start 65.04 75) (end 67.5 72.54) (width 0.25) (layer "B.Cu") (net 1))
 (segment (start 67.5 72.54) (end 67.5 72.5) (width 0.25) (layer "B.Cu") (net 1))
 (segment (start 72.5 67.5) (end 65.04 74.96) (width 0.25) (layer "B.Cu") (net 1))
 (segment (start 102.54 75) (end 105 72.54) (width 0.25) (layer "B.Cu") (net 1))
 (segment (start 105 72.5) (end 137.54 72.5) (width 0.25) (layer "B.Cu") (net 1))
 (segment (start 67.5 72.5) (end 105 72.5) (width 0.25) (layer "B.Cu") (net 1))
 (segment (start 105 72.54) (end 105 72.5) (width 0.25) (layer "B.Cu") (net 1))
 (segment (start 137.54 72.5) (end 140.04 75) (width 0.25) (layer "B.Cu") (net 1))
 (segment (start 65.04 74.96) (end 65.04 75) (width 0.25) (layer "B.Cu") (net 1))
 (segment (start 55 67.5) (end 67.42 67.5) (width 0.25) (layer "B.Cu") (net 2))
 (segment (start 220 65) (end 170.2 65) (width 0.25) (layer "F.Cu") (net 34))
 (segment (start 170.2 65) (end 165.2 60) (width 0.25) (layer "F.Cu") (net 34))
 (segment (start 211.274999 58.625001) (end 211.374999 58.625001) (width 0.25) (layer "B.Cu") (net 35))
 (segment (start 211.374999 58.625001) (end 212 58) (width 0.25) (layer "B.Cu") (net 35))
 (segment (start 209.9 60) (end 211.274999 58.625001) (width 0.25) (layer "B.Cu") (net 35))
 (segment (start 212 58) (end 247.5 58) (width 0.25) (layer "B.Cu") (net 35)))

